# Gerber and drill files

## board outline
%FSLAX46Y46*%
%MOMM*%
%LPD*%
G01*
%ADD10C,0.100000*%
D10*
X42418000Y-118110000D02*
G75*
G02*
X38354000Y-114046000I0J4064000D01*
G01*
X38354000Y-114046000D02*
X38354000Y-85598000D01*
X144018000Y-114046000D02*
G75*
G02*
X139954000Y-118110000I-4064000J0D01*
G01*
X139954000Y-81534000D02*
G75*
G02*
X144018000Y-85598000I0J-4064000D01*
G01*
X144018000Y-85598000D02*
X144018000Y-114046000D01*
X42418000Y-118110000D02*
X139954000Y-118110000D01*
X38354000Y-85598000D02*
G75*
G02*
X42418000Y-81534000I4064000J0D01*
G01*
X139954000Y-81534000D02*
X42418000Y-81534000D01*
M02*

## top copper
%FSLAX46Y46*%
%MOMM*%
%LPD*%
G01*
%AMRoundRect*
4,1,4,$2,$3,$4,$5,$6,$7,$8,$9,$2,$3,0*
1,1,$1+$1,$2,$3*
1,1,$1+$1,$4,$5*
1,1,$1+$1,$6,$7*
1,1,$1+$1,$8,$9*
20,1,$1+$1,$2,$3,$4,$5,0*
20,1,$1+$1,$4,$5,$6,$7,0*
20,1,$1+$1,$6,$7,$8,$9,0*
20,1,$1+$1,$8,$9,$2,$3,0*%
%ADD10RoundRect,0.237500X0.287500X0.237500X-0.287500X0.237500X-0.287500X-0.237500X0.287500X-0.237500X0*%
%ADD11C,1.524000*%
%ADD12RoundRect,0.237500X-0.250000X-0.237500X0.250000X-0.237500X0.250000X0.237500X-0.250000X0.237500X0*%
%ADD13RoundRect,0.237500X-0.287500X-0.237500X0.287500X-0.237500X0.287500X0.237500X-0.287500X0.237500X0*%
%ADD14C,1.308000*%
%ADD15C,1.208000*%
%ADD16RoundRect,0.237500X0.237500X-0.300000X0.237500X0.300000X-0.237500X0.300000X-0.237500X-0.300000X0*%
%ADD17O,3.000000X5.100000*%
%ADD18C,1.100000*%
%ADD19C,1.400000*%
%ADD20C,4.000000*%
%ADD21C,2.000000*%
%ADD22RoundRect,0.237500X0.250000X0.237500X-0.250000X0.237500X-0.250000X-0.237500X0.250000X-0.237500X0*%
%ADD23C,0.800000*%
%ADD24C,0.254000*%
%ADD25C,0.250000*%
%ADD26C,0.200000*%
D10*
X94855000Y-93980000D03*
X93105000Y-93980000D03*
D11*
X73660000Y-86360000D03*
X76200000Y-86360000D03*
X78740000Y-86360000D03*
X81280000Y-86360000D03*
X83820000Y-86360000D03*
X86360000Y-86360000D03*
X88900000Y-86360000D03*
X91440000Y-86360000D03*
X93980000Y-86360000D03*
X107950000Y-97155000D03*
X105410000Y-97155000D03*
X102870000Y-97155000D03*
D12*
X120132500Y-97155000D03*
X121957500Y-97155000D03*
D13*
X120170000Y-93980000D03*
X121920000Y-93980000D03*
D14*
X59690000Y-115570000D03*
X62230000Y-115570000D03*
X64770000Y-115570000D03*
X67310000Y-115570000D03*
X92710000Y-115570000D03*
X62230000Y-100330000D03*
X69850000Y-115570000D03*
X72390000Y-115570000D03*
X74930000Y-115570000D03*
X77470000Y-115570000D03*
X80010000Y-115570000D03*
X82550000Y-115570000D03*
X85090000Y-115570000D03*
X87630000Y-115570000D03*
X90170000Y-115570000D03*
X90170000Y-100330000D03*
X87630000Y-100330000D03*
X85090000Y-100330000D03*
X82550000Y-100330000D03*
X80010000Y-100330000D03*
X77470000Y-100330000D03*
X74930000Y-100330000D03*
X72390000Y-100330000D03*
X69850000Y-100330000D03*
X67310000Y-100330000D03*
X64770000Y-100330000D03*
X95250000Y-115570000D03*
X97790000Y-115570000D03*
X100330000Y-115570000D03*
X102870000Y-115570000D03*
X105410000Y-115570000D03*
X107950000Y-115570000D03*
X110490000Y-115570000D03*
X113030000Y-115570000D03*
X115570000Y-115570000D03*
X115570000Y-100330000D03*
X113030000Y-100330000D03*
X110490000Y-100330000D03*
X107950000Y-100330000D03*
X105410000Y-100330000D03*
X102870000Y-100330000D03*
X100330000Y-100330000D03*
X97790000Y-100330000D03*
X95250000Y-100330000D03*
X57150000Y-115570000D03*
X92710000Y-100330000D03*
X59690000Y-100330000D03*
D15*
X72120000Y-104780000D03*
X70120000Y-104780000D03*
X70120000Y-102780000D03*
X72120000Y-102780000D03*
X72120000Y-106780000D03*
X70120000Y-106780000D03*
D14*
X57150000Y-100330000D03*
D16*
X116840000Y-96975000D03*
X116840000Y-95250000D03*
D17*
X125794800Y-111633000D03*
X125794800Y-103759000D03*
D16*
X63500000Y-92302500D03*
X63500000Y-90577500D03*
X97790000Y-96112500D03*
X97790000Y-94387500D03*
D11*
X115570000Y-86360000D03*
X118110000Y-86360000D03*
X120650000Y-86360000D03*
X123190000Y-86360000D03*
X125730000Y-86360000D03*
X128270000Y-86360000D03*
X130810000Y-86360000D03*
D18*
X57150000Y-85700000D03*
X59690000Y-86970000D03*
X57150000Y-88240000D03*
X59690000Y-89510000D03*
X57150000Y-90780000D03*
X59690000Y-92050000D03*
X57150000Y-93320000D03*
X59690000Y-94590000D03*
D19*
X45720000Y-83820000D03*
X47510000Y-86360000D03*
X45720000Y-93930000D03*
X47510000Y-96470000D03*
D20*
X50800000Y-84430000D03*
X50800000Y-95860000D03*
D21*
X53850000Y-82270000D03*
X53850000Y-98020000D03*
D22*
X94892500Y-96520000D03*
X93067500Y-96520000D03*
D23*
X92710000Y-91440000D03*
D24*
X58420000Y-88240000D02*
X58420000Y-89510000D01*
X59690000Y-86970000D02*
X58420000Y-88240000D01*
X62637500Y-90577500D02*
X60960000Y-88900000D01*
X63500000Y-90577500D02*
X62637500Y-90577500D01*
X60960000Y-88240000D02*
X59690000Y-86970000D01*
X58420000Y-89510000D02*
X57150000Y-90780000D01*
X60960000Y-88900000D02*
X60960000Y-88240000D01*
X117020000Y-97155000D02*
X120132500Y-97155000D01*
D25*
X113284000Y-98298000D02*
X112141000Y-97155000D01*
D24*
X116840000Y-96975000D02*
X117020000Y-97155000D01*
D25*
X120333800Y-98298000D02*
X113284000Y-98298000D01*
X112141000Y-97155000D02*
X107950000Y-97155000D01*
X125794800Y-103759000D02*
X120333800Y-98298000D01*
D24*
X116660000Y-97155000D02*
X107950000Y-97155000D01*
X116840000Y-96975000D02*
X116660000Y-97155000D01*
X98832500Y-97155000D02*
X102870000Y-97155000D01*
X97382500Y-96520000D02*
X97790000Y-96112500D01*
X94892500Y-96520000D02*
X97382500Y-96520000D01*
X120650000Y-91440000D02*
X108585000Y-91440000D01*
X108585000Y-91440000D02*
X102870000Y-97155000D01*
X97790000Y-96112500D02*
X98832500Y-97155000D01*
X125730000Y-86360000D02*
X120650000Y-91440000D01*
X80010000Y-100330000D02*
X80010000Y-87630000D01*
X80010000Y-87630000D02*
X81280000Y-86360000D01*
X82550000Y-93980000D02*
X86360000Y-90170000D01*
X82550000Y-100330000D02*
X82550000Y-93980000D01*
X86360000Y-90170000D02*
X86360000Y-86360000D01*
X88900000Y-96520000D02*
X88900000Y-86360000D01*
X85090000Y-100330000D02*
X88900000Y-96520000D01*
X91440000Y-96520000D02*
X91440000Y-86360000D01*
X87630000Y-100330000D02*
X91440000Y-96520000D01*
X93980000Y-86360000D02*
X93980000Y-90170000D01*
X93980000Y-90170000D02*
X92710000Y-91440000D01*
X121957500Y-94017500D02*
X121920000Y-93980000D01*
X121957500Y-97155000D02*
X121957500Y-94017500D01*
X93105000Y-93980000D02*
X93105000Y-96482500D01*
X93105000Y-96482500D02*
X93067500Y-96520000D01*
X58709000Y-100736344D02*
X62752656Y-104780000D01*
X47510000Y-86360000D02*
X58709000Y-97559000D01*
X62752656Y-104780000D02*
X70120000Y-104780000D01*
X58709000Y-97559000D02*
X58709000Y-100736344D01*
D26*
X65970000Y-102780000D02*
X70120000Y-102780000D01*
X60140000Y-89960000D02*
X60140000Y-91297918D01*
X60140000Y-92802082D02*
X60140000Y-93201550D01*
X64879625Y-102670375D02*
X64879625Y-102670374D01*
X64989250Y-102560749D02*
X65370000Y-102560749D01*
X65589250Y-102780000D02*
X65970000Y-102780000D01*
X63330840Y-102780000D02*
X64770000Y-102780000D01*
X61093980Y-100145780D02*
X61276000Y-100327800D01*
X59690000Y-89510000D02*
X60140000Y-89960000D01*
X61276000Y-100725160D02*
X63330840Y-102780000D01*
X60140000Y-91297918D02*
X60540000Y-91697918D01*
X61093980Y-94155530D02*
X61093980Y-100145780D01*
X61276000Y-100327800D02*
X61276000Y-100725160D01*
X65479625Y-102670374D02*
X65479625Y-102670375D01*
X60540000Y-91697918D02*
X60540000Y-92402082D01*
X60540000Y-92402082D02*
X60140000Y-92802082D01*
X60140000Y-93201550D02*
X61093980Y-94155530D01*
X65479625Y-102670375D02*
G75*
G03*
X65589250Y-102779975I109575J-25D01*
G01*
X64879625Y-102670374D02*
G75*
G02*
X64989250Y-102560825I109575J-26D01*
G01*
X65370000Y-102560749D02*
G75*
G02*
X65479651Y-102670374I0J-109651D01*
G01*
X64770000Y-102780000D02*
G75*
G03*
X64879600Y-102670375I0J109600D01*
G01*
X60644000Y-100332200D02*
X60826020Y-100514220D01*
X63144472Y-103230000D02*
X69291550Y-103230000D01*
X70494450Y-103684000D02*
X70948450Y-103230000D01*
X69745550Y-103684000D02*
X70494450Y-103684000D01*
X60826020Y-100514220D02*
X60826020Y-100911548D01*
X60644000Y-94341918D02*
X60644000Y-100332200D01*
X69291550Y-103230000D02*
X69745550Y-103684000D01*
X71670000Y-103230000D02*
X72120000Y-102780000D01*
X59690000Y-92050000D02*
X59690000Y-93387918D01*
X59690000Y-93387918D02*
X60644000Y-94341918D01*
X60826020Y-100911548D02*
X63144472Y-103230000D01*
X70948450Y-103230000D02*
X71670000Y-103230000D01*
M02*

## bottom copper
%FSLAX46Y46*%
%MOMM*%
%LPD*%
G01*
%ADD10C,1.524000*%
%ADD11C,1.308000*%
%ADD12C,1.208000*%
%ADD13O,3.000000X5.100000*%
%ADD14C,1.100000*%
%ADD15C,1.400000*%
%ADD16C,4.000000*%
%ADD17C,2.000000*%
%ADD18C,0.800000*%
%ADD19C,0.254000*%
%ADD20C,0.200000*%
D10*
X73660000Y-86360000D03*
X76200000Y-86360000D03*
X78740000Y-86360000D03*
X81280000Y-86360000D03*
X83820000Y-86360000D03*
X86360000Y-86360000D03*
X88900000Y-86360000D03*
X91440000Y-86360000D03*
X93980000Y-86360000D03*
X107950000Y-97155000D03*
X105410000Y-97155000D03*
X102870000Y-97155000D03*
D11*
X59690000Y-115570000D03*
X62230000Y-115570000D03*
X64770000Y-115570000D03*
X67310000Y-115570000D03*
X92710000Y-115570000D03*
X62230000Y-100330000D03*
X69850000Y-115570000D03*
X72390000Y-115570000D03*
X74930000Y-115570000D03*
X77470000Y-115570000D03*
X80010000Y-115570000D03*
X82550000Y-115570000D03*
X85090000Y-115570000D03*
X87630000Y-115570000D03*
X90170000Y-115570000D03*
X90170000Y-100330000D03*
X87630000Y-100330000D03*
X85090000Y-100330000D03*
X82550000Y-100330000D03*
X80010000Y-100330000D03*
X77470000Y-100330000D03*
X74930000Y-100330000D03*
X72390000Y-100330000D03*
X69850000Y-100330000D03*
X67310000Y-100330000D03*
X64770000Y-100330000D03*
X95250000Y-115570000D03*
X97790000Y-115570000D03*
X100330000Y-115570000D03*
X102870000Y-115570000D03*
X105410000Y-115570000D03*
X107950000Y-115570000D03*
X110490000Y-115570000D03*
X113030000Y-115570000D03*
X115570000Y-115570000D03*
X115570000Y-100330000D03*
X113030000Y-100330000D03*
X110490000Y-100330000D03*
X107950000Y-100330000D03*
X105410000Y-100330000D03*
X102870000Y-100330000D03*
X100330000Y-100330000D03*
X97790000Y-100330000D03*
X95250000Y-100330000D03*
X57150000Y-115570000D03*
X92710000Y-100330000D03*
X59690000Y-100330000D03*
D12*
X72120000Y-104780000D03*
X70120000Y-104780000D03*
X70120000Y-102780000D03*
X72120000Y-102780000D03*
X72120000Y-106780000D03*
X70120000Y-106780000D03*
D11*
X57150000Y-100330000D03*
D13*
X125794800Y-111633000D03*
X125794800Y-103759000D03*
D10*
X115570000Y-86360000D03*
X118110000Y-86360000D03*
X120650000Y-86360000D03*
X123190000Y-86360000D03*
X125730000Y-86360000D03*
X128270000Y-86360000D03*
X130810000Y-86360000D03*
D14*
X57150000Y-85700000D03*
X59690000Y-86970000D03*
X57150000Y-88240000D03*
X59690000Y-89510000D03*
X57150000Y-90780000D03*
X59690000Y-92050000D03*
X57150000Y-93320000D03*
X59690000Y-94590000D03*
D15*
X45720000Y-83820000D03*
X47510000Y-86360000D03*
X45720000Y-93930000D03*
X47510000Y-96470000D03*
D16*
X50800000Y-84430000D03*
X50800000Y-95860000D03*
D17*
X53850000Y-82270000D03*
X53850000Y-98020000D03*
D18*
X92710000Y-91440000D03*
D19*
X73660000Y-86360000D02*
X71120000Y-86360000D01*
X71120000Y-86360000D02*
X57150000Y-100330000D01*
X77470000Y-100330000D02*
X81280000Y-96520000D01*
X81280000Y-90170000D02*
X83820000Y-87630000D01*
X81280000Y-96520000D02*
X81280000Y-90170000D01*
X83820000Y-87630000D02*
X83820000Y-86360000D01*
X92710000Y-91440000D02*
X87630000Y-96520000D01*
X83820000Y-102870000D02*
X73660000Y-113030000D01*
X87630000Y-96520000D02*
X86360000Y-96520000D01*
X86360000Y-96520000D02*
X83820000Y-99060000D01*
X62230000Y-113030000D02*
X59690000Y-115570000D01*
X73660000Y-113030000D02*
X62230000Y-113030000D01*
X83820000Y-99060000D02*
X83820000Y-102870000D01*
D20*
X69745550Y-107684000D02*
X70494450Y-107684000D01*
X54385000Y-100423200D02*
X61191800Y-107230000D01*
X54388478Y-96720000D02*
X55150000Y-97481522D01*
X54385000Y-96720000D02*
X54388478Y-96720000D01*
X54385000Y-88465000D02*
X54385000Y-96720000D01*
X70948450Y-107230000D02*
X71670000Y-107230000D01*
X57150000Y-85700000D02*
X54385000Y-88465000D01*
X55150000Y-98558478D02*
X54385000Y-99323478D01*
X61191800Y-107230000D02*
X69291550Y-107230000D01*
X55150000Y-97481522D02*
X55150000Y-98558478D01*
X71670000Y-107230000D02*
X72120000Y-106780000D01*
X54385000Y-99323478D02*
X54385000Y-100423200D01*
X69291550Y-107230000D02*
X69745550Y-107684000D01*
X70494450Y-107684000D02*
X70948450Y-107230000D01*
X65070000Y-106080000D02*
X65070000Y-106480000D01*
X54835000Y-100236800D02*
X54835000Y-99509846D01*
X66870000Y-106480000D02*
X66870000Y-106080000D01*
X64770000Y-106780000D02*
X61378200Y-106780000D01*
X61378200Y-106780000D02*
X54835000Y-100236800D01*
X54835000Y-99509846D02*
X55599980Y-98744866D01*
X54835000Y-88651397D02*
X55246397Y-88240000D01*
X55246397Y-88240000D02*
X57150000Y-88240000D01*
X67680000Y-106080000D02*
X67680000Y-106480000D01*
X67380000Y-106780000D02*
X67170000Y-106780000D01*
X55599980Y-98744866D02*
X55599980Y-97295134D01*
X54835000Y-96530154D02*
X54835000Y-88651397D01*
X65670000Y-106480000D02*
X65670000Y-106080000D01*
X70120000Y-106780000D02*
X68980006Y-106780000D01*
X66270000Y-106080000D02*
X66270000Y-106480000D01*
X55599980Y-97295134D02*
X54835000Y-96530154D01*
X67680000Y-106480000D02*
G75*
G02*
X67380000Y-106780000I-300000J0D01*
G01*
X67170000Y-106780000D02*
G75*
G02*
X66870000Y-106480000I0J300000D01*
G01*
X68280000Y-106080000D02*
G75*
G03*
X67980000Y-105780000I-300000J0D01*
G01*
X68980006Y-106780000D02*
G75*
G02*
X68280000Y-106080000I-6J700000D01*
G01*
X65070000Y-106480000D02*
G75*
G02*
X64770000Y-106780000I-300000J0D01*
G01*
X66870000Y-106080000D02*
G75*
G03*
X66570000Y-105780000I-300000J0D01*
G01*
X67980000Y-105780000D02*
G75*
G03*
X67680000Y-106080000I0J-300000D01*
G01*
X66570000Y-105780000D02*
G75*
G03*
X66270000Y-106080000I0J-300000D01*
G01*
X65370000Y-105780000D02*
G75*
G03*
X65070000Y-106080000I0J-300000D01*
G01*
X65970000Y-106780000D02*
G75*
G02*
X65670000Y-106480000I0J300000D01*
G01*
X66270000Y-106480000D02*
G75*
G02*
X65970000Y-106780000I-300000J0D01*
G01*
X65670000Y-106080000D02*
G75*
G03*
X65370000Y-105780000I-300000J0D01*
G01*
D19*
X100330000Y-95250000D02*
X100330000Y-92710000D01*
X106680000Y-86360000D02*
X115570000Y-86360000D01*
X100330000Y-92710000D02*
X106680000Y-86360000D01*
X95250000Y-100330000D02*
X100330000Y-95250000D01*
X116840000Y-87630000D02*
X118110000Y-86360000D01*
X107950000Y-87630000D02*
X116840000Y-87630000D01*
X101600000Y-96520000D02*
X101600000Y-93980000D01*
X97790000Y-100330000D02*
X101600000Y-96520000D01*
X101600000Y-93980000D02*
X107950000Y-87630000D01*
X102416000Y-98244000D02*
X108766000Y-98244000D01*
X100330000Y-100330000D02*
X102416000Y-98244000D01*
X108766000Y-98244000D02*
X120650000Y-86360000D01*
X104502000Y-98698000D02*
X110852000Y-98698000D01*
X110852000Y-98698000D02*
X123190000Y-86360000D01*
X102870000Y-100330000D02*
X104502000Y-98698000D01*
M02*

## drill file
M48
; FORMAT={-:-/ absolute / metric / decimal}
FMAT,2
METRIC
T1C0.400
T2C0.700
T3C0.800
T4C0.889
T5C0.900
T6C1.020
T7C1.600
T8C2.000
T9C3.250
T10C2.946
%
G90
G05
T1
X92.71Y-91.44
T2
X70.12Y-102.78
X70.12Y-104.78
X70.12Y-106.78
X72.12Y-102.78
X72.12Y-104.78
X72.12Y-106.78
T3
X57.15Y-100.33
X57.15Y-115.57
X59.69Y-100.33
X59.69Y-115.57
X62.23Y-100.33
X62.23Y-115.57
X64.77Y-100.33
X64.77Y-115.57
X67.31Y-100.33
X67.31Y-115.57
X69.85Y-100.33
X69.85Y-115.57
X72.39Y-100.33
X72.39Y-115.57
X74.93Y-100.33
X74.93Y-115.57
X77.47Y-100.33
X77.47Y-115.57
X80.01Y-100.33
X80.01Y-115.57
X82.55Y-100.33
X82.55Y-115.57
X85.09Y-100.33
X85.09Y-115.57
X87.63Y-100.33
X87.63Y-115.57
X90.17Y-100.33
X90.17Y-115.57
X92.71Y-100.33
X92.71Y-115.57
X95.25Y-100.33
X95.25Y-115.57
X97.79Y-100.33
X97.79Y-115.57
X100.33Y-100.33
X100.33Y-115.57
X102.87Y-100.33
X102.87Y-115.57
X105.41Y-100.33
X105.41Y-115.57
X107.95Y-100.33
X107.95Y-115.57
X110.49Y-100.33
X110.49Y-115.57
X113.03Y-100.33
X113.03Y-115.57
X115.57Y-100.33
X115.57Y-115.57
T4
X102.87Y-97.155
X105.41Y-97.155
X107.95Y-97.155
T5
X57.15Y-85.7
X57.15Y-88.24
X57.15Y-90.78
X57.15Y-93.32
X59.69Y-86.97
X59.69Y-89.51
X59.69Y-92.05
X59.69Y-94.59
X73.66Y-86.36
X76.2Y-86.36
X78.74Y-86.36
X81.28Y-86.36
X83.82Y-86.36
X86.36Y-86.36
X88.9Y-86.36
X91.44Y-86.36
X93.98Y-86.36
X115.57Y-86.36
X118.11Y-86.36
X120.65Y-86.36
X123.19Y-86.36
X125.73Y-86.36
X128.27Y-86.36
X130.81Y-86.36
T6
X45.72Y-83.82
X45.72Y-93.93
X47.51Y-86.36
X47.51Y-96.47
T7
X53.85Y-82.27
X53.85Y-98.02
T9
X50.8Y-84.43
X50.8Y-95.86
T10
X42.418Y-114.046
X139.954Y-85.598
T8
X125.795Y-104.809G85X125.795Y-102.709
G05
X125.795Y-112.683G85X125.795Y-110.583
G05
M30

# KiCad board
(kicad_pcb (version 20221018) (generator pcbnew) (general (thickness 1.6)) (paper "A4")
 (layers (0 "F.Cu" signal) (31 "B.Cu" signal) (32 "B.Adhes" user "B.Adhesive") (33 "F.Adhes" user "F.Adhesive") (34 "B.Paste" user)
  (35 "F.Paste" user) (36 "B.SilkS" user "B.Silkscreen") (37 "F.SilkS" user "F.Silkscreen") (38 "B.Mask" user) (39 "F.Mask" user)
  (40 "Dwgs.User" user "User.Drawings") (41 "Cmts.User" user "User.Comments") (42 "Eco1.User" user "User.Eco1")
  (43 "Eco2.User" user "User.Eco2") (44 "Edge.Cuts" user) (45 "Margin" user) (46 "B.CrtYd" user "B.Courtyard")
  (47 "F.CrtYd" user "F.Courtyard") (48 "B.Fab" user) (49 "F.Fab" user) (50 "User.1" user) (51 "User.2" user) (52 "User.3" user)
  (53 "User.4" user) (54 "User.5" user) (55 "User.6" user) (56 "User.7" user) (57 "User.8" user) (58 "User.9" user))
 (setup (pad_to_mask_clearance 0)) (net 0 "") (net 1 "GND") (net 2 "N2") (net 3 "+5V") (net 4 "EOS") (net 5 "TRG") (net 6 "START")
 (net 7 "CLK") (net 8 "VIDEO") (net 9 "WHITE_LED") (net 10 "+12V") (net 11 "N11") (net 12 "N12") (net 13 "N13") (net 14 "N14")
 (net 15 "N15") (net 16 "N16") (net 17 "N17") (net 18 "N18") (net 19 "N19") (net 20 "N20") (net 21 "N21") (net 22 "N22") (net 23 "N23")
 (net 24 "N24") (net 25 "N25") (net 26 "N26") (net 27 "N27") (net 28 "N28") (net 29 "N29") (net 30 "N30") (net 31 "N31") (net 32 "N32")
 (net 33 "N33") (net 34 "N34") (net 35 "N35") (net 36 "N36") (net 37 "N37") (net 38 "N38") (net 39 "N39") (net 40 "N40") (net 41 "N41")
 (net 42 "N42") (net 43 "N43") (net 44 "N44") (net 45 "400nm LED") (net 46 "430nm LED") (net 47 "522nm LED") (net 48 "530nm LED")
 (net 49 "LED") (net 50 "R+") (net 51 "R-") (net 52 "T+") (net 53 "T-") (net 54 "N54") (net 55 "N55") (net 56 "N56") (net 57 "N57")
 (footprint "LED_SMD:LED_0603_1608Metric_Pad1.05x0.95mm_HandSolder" (layer "F.Cu") (at 93.98 93.98 180)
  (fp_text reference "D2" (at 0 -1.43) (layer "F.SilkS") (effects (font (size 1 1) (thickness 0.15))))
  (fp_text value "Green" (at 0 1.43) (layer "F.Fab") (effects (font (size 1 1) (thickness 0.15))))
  (pad "1" smd roundrect (at -0.875 0 180) (size 1.05 0.95) (layers "F.Cu" "F.Paste" "F.Mask") (roundrect_rratio 0.25) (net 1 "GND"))
  (pad "2" smd roundrect (at 0.875 0 180) (size 1.05 0.95) (layers "F.Cu" "F.Paste" "F.Mask") (roundrect_rratio 0.25) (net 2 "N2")))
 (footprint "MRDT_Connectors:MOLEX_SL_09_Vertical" (layer "F.Cu") (at 73.66 86.36)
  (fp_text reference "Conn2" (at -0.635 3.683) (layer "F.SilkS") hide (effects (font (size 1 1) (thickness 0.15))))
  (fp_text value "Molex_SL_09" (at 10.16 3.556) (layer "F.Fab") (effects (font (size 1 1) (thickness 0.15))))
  (pad "1" thru_hole circle (at 0 0) (size 1.524 1.524) (drill 0.9) (layers "*.Cu" "*.Mask") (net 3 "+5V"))
  (pad "2" thru_hole circle (at 2.54 0) (size 1.524 1.524) (drill 0.9) (layers "*.Cu" "*.Mask") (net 1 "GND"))
  (pad "3" thru_hole circle (at 5.08 0) (size 1.524 1.524) (drill 0.9) (layers "*.Cu" "*.Mask") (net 1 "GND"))
  (pad "4" thru_hole circle (at 7.62 0) (size 1.524 1.524) (drill 0.9) (layers "*.Cu" "*.Mask") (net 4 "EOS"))
  (pad "5" thru_hole circle (at 10.16 0) (size 1.524 1.524) (drill 0.9) (layers "*.Cu" "*.Mask") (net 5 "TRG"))
  (pad "6" thru_hole circle (at 12.7 0) (size 1.524 1.524) (drill 0.9) (layers "*.Cu" "*.Mask") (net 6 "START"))
  (pad "7" thru_hole circle (at 15.24 0) (size 1.524 1.524) (drill 0.9) (layers "*.Cu" "*.Mask") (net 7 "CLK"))
  (pad "8" thru_hole circle (at 17.78 0) (size 1.524 1.524) (drill 0.9) (layers "*.Cu" "*.Mask") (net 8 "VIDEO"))
  (pad "9" thru_hole circle (at 20.32 0) (size 1.524 1.524) (drill 0.9) (layers "*.Cu" "*.Mask") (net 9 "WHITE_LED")))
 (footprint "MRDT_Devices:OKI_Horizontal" (layer "F.Cu") (at 107.95 97.155 180)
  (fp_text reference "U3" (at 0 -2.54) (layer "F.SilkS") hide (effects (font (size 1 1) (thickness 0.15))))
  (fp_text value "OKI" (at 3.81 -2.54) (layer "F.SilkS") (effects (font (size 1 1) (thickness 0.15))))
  (pad "1" thru_hole circle (at 0 0 180) (size 1.524 1.524) (drill 0.889) (layers "*.Cu" "*.Mask") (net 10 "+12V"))
  (pad "2" thru_hole circle (at 2.54 0 180) (size 1.524 1.524) (drill 0.889) (layers "*.Cu" "*.Mask") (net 1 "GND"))
  (pad "3" thru_hole circle (at 5.08 0 180) (size 1.524 1.524) (drill 0.889) (layers "*.Cu" "*.Mask") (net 3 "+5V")))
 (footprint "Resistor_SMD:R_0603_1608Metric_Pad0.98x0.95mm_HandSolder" (layer "F.Cu") (at 121.045 97.155)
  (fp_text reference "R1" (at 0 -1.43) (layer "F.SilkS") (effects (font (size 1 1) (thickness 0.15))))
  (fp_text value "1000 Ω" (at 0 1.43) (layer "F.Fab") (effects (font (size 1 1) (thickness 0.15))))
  (pad "1" smd roundrect (at -0.9125 0) (size 0.975 0.95) (layers "F.Cu" "F.Paste" "F.Mask") (roundrect_rratio 0.25) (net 10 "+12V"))
  (pad "2" smd roundrect (at 0.9125 0) (size 0.975 0.95) (layers "F.Cu" "F.Paste" "F.Mask") (roundrect_rratio 0.25) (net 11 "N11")))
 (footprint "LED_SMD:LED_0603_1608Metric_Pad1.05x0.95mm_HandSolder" (layer "F.Cu") (at 121.045 93.98)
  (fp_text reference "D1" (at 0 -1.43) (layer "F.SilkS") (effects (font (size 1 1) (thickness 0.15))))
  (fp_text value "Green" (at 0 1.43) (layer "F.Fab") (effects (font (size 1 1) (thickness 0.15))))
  (pad "1" smd roundrect (at -0.875 0) (size 1.05 0.95) (layers "F.Cu" "F.Paste" "F.Mask") (roundrect_rratio 0.25) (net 1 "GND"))
  (pad "2" smd roundrect (at 0.875 0) (size 1.05 0.95) (layers "F.Cu" "F.Paste" "F.Mask") (roundrect_rratio 0.25) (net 11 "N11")))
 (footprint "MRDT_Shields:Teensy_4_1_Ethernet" (layer "F.Cu") (at 86.36 107.95)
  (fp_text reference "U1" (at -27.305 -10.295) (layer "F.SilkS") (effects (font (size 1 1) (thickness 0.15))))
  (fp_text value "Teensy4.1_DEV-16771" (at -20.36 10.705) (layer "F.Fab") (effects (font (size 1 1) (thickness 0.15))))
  (pad "0" thru_hole circle (at -26.67 7.62) (size 1.308 1.308) (drill 0.8) (layers "*.Cu" "*.Mask") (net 9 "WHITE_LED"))
  (pad "1" thru_hole circle (at -24.13 7.62) (size 1.308 1.308) (drill 0.8) (layers "*.Cu" "*.Mask") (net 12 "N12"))
  (pad "2" thru_hole circle (at -21.59 7.62) (size 1.308 1.308) (drill 0.8) (layers "*.Cu" "*.Mask") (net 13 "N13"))
  (pad "3" thru_hole circle (at -19.05 7.62) (size 1.308 1.308) (drill 0.8) (layers "*.Cu" "*.Mask") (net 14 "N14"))
  (pad "3.3V_1" thru_hole circle (at 6.35 7.62) (size 1.308 1.308) (drill 0.8) (layers "*.Cu" "*.Mask") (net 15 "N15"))
  (pad "3.3V_2" thru_hole circle (at -24.13 -7.62) (size 1.308 1.308) (drill 0.8) (layers "*.Cu" "*.Mask") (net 15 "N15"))
  (pad "4" thru_hole circle (at -16.51 7.62) (size 1.308 1.308) (drill 0.8) (layers "*.Cu" "*.Mask") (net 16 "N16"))
  (pad "5" thru_hole circle (at -13.97 7.62) (size 1.308 1.308) (drill 0.8) (layers "*.Cu" "*.Mask") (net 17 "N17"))
  (pad "6" thru_hole circle (at -11.43 7.62) (size 1.308 1.308) (drill 0.8) (layers "*.Cu" "*.Mask") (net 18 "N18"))
  (pad "7" thru_hole circle (at -8.89 7.62) (size 1.308 1.308) (drill 0.8) (layers "*.Cu" "*.Mask") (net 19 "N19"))
  (pad "8" thru_hole circle (at -6.35 7.62) (size 1.308 1.308) (drill 0.8) (layers "*.Cu" "*.Mask") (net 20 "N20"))
  (pad "9" thru_hole circle (at -3.81 7.62) (size 1.308 1.308) (drill 0.8) (layers "*.Cu" "*.Mask") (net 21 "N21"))
  (pad "10" thru_hole circle (at -1.27 7.62) (size 1.308 1.308) (drill 0.8) (layers "*.Cu" "*.Mask") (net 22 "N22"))
  (pad "11" thru_hole circle (at 1.27 7.62) (size 1.308 1.308) (drill 0.8) (layers "*.Cu" "*.Mask") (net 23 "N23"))
  (pad "12" thru_hole circle (at 3.81 7.62) (size 1.308 1.308) (drill 0.8) (layers "*.Cu" "*.Mask") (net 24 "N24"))
  (pad "13" thru_hole circle (at 3.81 -7.62) (size 1.308 1.308) (drill 0.8) (layers "*.Cu" "*.Mask") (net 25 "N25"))
  (pad "14" thru_hole circle (at 1.27 -7.62) (size 1.308 1.308) (drill 0.8) (layers "*.Cu" "*.Mask") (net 8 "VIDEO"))
  (pad "15" thru_hole circle (at -1.27 -7.62) (size 1.308 1.308) (drill 0.8) (layers "*.Cu" "*.Mask") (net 7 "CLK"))
  (pad "16" thru_hole circle (at -3.81 -7.62) (size 1.308 1.308) (drill 0.8) (layers "*.Cu" "*.Mask") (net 6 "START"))
  (pad "17" thru_hole circle (at -6.35 -7.62) (size 1.308 1.308) (drill 0.8) (layers "*.Cu" "*.Mask") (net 4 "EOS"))
  (pad "18" thru_hole circle (at -8.89 -7.62) (size 1.308 1.308) (drill 0.8) (layers "*.Cu" "*.Mask") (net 5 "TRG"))
  (pad "19" thru_hole circle (at -11.43 -7.62) (size 1.308 1.308) (drill 0.8) (layers "*.Cu" "*.Mask") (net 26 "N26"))
  (pad "20" thru_hole circle (at -13.97 -7.62) (size 1.308 1.308) (drill 0.8) (layers "*.Cu" "*.Mask") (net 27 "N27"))
  (pad "21" thru_hole circle (at -16.51 -7.62) (size 1.308 1.308) (drill 0.8) (layers "*.Cu" "*.Mask") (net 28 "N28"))
  (pad "22" thru_hole circle (at -19.05 -7.62) (size 1.308 1.308) (drill 0.8) (layers "*.Cu" "*.Mask") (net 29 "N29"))
  (pad "23" thru_hole circle (at -21.59 -7.62) (size 1.308 1.308) (drill 0.8) (layers "*.Cu" "*.Mask") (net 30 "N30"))
  (pad "24" thru_hole circle (at 8.89 7.62) (size 1.308 1.308) (drill 0.8) (layers "*.Cu" "*.Mask") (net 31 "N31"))
  (pad "25" thru_hole circle (at 11.43 7.62) (size 1.308 1.308) (drill 0.8) (layers "*.Cu" "*.Mask") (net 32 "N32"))
  (pad "26" thru_hole circle (at 13.97 7.62) (size 1.308 1.308) (drill 0.8) (layers "*.Cu" "*.Mask") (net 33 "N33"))
  (pad "27" thru_hole circle (at 16.51 7.62) (size 1.308 1.308) (drill 0.8) (layers "*.Cu" "*.Mask") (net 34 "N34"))
  (pad "28" thru_hole circle (at 19.05 7.62) (size 1.308 1.308) (drill 0.8) (layers "*.Cu" "*.Mask") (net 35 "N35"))
  (pad "29" thru_hole circle (at 21.59 7.62) (size 1.308 1.308) (drill 0.8) (layers "*.Cu" "*.Mask") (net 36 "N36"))
  (pad "30" thru_hole circle (at 24.13 7.62) (size 1.308 1.308) (drill 0.8) (layers "*.Cu" "*.Mask") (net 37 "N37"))
  (pad "31" thru_hole circle (at 26.67 7.62) (size 1.308 1.308) (drill 0.8) (layers "*.Cu" "*.Mask") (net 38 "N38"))
  (pad "32" thru_hole circle (at 29.21 7.62) (size 1.308 1.308) (drill 0.8) (layers "*.Cu" "*.Mask") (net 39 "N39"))
  (pad "33" thru_hole circle (at 29.21 -7.62) (size 1.308 1.308) (drill 0.8) (layers "*.Cu" "*.Mask") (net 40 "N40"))
  (pad "34" thru_hole circle (at 26.67 -7.62) (size 1.308 1.308) (drill 0.8) (layers "*.Cu" "*.Mask") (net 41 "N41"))
  (pad "35" thru_hole circle (at 24.13 -7.62) (size 1.308 1.308) (drill 0.8) (layers "*.Cu" "*.Mask") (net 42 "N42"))
  (pad "36" thru_hole circle (at 21.59 -7.62) (size 1.308 1.308) (drill 0.8) (layers "*.Cu" "*.Mask") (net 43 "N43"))
  (pad "37" thru_hole circle (at 19.05 -7.62) (size 1.308 1.308) (drill 0.8) (layers "*.Cu" "*.Mask") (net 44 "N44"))
  (pad "38" thru_hole circle (at 16.51 -7.62) (size 1.308 1.308) (drill 0.8) (layers "*.Cu" "*.Mask") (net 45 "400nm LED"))
  (pad "39" thru_hole circle (at 13.97 -7.62) (size 1.308 1.308) (drill 0.8) (layers "*.Cu" "*.Mask") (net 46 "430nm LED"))
  (pad "40" thru_hole circle (at 11.43 -7.62) (size 1.308 1.308) (drill 0.8) (layers "*.Cu" "*.Mask") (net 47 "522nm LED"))
  (pad "41" thru_hole circle (at 8.89 -7.62) (size 1.308 1.308) (drill 0.8) (layers "*.Cu" "*.Mask") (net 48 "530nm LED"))
  (pad "GND1" thru_hole circle (at -29.21 7.62) (size 1.308 1.308) (drill 0.8) (layers "*.Cu" "*.Mask") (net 1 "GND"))
  (pad "GND2" thru_hole circle (at 6.35 -7.62) (size 1.308 1.308) (drill 0.8) (layers "*.Cu" "*.Mask") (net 1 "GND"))
  (pad "GND3" thru_hole circle (at -26.67 -7.62) (size 1.308 1.308) (drill 0.8) (layers "*.Cu" "*.Mask") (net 1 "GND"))
  (pad "GND5" thru_hole circle (at -14.24 -3.17) (size 1.208 1.208) (drill 0.7) (layers "*.Cu" "*.Mask") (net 1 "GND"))
  (pad "LED" thru_hole circle (at -16.24 -3.17) (size 1.208 1.208) (drill 0.7) (layers "*.Cu" "*.Mask") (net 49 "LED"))
  (pad "R+" thru_hole circle (at -16.24 -5.17) (size 1.208 1.208) (drill 0.7) (layers "*.Cu" "*.Mask") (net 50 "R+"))
  (pad "R-" thru_hole circle (at -14.24 -5.17) (size 1.208 1.208) (drill 0.7) (layers "*.Cu" "*.Mask") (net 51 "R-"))
  (pad "T+" thru_hole circle (at -14.24 -1.17) (size 1.208 1.208) (drill 0.7) (layers "*.Cu" "*.Mask") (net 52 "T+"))
  (pad "T-" thru_hole circle (at -16.24 -1.17) (size 1.208 1.208) (drill 0.7) (layers "*.Cu" "*.Mask") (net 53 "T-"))
  (pad "VIN" thru_hole circle (at -29.21 -7.62) (size 1.308 1.308) (drill 0.8) (layers "*.Cu" "*.Mask") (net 3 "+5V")))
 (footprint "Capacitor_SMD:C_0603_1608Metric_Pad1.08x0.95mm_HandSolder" (layer "F.Cu") (at 116.84 96.1125 90)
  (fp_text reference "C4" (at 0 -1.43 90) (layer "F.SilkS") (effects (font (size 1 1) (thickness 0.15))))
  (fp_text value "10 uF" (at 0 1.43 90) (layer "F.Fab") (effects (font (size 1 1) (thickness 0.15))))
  (pad "1" smd roundrect (at -0.8625 0 90) (size 1.075 0.95) (layers "F.Cu" "F.Paste" "F.Mask") (roundrect_rratio 0.25) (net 10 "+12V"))
  (pad "2" smd roundrect (at 0.8625 0 90) (size 1.075 0.95) (layers "F.Cu" "F.Paste" "F.Mask") (roundrect_rratio 0.25) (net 1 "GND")))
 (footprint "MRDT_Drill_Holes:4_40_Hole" (layer "F.Cu") (at 139.954 85.598) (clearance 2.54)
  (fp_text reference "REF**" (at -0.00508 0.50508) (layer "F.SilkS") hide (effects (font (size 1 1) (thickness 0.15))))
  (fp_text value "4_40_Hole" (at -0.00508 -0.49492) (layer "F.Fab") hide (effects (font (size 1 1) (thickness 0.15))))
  (pad "" np_thru_hole circle (at 0 0) (size 2.9464 2.9464) (drill 2.9464) (layers "*.Cu" "*.Mask") (clearance 2.5)))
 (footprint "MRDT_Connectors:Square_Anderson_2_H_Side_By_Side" (layer "F.Cu") (at 125.4202 112.183 180)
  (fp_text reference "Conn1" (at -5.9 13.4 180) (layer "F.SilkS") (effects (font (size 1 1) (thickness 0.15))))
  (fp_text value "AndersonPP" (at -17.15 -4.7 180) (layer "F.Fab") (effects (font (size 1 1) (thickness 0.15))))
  (pad "1" thru_hole oval (at -0.3746 0.55 180) (size 3 5.1) (drill oval 2 4.1) (layers "*.Cu" "*.Mask" "F.Paste") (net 1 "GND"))
  (pad "2" thru_hole oval (at -0.3746 8.424 180) (size 3 5.1) (drill oval 2 4.1) (layers "*.Cu" "*.Mask" "F.Paste") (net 10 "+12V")))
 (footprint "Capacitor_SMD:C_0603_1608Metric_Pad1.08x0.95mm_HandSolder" (layer "F.Cu") (at 63.5 91.44 90)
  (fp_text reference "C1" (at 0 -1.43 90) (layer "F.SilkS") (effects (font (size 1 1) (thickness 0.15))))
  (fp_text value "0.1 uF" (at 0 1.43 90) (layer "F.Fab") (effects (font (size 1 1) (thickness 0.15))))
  (pad "1" smd roundrect (at -0.8625 0 90) (size 1.075 0.95) (layers "F.Cu" "F.Paste" "F.Mask") (roundrect_rratio 0.25) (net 1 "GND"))
  (pad "2" smd roundrect (at 0.8625 0 90) (size 1.075 0.95) (layers "F.Cu" "F.Paste" "F.Mask") (roundrect_rratio 0.25) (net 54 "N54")))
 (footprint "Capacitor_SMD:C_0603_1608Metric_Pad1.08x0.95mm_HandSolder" (layer "F.Cu") (at 97.79 95.25 90)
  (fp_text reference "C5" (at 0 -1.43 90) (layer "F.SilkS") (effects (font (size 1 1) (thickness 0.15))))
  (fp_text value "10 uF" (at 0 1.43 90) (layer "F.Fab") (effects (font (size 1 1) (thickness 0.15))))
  (pad "1" smd roundrect (at -0.8625 0 90) (size 1.075 0.95) (layers "F.Cu" "F.Paste" "F.Mask") (roundrect_rratio 0.25) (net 3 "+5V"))
  (pad "2" smd roundrect (at 0.8625 0 90) (size 1.075 0.95) (layers "F.Cu" "F.Paste" "F.Mask") (roundrect_rratio 0.25) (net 1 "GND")))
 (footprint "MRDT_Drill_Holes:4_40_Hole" (layer "F.Cu") (at 42.418 114.046) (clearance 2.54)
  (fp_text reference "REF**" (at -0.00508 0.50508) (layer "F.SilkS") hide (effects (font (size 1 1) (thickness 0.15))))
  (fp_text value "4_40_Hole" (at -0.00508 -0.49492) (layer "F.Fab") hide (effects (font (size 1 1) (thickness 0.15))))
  (pad "" np_thru_hole circle (at 0 0) (size 2.9464 2.9464) (drill 2.9464) (layers "*.Cu" "*.Mask") (clearance 2.5)))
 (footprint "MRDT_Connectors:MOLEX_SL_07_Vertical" (layer "F.Cu") (at 115.57 86.36)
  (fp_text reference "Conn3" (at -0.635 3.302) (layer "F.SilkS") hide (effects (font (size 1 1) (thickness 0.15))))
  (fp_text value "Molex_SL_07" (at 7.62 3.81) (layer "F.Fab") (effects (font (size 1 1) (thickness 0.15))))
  (pad "1" thru_hole circle (at 0 0) (size 1.524 1.524) (drill 0.9) (layers "*.Cu" "*.Mask") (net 48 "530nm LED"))
  (pad "2" thru_hole circle (at 2.54 0) (size 1.524 1.524) (drill 0.9) (layers "*.Cu" "*.Mask") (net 47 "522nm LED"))
  (pad "3" thru_hole circle (at 5.08 0) (size 1.524 1.524) (drill 0.9) (layers "*.Cu" "*.Mask") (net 46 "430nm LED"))
  (pad "4" thru_hole circle (at 7.62 0) (size 1.524 1.524) (drill 0.9) (layers "*.Cu" "*.Mask") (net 45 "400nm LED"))
  (pad "5" thru_hole circle (at 10.16 0) (size 1.524 1.524) (drill 0.9) (layers "*.Cu" "*.Mask") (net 3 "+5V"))
  (pad "6" thru_hole circle (at 12.7 0) (size 1.524 1.524) (drill 0.9) (layers "*.Cu" "*.Mask") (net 1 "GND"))
  (pad "7" thru_hole circle (at 15.24 0) (size 1.524 1.524) (drill 0.9) (layers "*.Cu" "*.Mask") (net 1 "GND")))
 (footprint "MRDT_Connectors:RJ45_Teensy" (layer "F.Cu") (at 37.8 90.27 -90)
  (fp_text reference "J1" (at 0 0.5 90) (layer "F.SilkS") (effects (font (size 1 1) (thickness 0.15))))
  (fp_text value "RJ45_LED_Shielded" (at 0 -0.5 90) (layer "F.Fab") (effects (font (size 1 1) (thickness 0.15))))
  (pad "1" thru_hole circle (at -4.57 -19.35 270) (size 1.1 1.1) (drill 0.9) (layers "*.Cu" "*.Mask") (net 52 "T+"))
  (pad "2" thru_hole circle (at -3.3 -21.89 270) (size 1.1 1.1) (drill 0.9) (layers "*.Cu" "*.Mask") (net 54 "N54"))
  (pad "3" thru_hole circle (at -2.03 -19.35 270) (size 1.1 1.1) (drill 0.9) (layers "*.Cu" "*.Mask") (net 53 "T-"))
  (pad "4" thru_hole circle (at -0.76 -21.89 270) (size 1.1 1.1) (drill 0.9) (layers "*.Cu" "*.Mask") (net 50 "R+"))
  (pad "5" thru_hole circle (at 0.51 -19.35 270) (size 1.1 1.1) (drill 0.9) (layers "*.Cu" "*.Mask") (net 54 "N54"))
  (pad "6" thru_hole circle (at 1.78 -21.89 270) (size 1.1 1.1) (drill 0.9) (layers "*.Cu" "*.Mask") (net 51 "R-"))
  (pad "7" thru_hole circle (at 3.05 -19.35 270) (size 1.1 1.1) (drill 0.9) (layers "*.Cu" "*.Mask") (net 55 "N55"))
  (pad "8" thru_hole circle (at 4.32 -21.89 270) (size 1.1 1.1) (drill 0.9) (layers "*.Cu" "*.Mask") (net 1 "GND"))
  (pad "9" thru_hole circle (at -6.45 -7.92 270) (size 1.4 1.4) (drill 1.02) (layers "*.Cu" "*.Mask") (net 1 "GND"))
  (pad "10" thru_hole circle (at -3.91 -9.71 270) (size 1.4 1.4) (drill 1.02) (layers "*.Cu" "*.Mask") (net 49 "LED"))
  (pad "11" thru_hole circle (at 3.66 -7.92 270) (size 1.4 1.4) (drill 1.02) (layers "*.Cu" "*.Mask") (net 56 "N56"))
  (pad "12" thru_hole circle (at 6.2 -9.71 270) (size 1.4 1.4) (drill 1.02) (layers "*.Cu" "*.Mask") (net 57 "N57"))
  (pad "13" thru_hole circle (at -5.84 -13 270) (size 4 4) (drill 3.25) (layers "*.Cu" "*.Mask"))
  (pad "14" thru_hole circle (at 5.59 -13 270) (size 4 4) (drill 3.25) (layers "*.Cu" "*.Mask"))
  (pad "SH" thru_hole circle (at -8 -16.05 270) (size 2 2) (drill 1.6) (layers "*.Cu" "*.Mask") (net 1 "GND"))
  (pad "SH" thru_hole circle (at 7.75 -16.05 270) (size 2 2) (drill 1.6) (layers "*.Cu" "*.Mask") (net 1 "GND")))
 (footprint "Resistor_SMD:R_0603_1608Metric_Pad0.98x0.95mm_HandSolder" (layer "F.Cu") (at 93.98 96.52 180)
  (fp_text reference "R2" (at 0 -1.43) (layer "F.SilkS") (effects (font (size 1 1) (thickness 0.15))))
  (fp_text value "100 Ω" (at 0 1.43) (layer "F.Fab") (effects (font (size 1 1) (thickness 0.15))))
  (pad "1" smd roundrect (at -0.9125 0 180) (size 0.975 0.95) (layers "F.Cu" "F.Paste" "F.Mask") (roundrect_rratio 0.25) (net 3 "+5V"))
  (pad "2" smd roundrect (at 0.9125 0 180) (size 0.975 0.95) (layers "F.Cu" "F.Paste" "F.Mask") (roundrect_rratio 0.25) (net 2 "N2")))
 (gr_arc (start 42.418 118.11) (mid 39.544318 116.919682) (end 38.354 114.046) (stroke (width 0.1) (type default)) (layer "Edge.Cuts"))
 (gr_line (start 38.354 114.046) (end 38.354 85.598) (stroke (width 0.1) (type default)) (layer "Edge.Cuts"))
 (gr_arc (start 144.018 114.046) (mid 142.827683 116.919683) (end 139.954 118.11) (stroke (width 0.1) (type default)) (layer "Edge.Cuts"))
 (gr_arc (start 139.954 81.534) (mid 142.827682 82.724318) (end 144.018 85.598) (stroke (width 0.1) (type default)) (layer "Edge.Cuts"))
 (gr_line (start 144.018 85.598) (end 144.018 114.046) (stroke (width 0.1) (type default)) (layer "Edge.Cuts"))
 (gr_line (start 42.418 118.11) (end 139.954 118.11) (stroke (width 0.1) (type default)) (layer "Edge.Cuts"))
 (gr_arc (start 38.354 85.598) (mid 39.544317 82.724317) (end 42.418 81.534) (stroke (width 0.1) (type default)) (layer "Edge.Cuts"))
 (gr_line (start 139.954 81.534) (end 42.418 81.534) (stroke (width 0.1) (type default)) (layer "Edge.Cuts"))
 (segment (start 58.42 88.24) (end 58.42 89.51) (width 0.254) (layer "F.Cu") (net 54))
 (segment (start 59.69 86.97) (end 58.42 88.24) (width 0.254) (layer "F.Cu") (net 54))
 (segment (start 62.6375 90.5775) (end 60.96 88.9) (width 0.254) (layer "F.Cu") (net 54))
 (segment (start 63.5 90.5775) (end 62.6375 90.5775) (width 0.254) (layer "F.Cu") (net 54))
 (segment (start 60.96 88.24) (end 59.69 86.97) (width 0.254) (layer "F.Cu") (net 54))
 (segment (start 58.42 89.51) (end 57.15 90.78) (width 0.254) (layer "F.Cu") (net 54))
 (segment (start 60.96 88.9) (end 60.96 88.24) (width 0.254) (layer "F.Cu") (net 54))
 (segment (start 117.02 97.155) (end 120.1325 97.155) (width 0.254) (layer "F.Cu") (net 10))
 (segment (start 113.284 98.298) (end 112.141 97.155) (width 0.25) (layer "F.Cu") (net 10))
 (segment (start 116.84 96.975) (end 117.02 97.155) (width 0.254) (layer "F.Cu") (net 10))
 (segment (start 120.3338 98.298) (end 113.284 98.298) (width 0.25) (layer "F.Cu") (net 10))
 (segment (start 112.141 97.155) (end 107.95 97.155) (width 0.25) (layer "F.Cu") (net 10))
 (segment (start 125.7948 103.759) (end 120.3338 98.298) (width 0.25) (layer "F.Cu") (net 10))
 (segment (start 116.66 97.155) (end 107.95 97.155) (width 0.254) (layer "F.Cu") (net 10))
 (segment (start 116.84 96.975) (end 116.66 97.155) (width 0.254) (layer "F.Cu") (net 10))
 (segment (start 98.8325 97.155) (end 102.87 97.155) (width 0.254) (layer "F.Cu") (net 3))
 (segment (start 97.3825 96.52) (end 97.79 96.1125) (width 0.254) (layer "F.Cu") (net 3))
 (segment (start 94.8925 96.52) (end 97.3825 96.52) (width 0.254) (layer "F.Cu") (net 3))
 (segment (start 120.65 91.44) (end 108.585 91.44) (width 0.254) (layer "F.Cu") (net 3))
 (segment (start 108.585 91.44) (end 102.87 97.155) (width 0.254) (layer "F.Cu") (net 3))
 (segment (start 97.79 96.1125) (end 98.8325 97.155) (width 0.254) (layer "F.Cu") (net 3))
 (segment (start 125.73 86.36) (end 120.65 91.44) (width 0.254) (layer "F.Cu") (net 3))
 (segment (start 73.66 86.36) (end 71.12 86.36) (width 0.254) (layer "B.Cu") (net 3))
 (segment (start 71.12 86.36) (end 57.15 100.33) (width 0.254) (layer "B.Cu") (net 3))
 (segment (start 80.01 100.33) (end 80.01 87.63) (width 0.254) (layer "F.Cu") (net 4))
 (segment (start 80.01 87.63) (end 81.28 86.36) (width 0.254) (layer "F.Cu") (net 4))
 (segment (start 77.47 100.33) (end 81.28 96.52) (width 0.254) (layer "B.Cu") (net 5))
 (segment (start 81.28 90.17) (end 83.82 87.63) (width 0.254) (layer "B.Cu") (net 5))
 (segment (start 81.28 96.52) (end 81.28 90.17) (width 0.254) (layer "B.Cu") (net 5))
 (segment (start 83.82 87.63) (end 83.82 86.36) (width 0.254) (layer "B.Cu") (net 5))
 (segment (start 82.55 93.98) (end 86.36 90.17) (width 0.254) (layer "F.Cu") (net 6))
 (segment (start 82.55 100.33) (end 82.55 93.98) (width 0.254) (layer "F.Cu") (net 6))
 (segment (start 86.36 90.17) (end 86.36 86.36) (width 0.254) (layer "F.Cu") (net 6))
 (segment (start 88.9 96.52) (end 88.9 86.36) (width 0.254) (layer "F.Cu") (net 7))
 (segment (start 85.09 100.33) (end 88.9 96.52) (width 0.254) (layer "F.Cu") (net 7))
 (segment (start 91.44 96.52) (end 91.44 86.36) (width 0.254) (layer "F.Cu") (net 8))
 (segment (start 87.63 100.33) (end 91.44 96.52) (width 0.254) (layer "F.Cu") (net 8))
 (segment (start 93.98 86.36) (end 93.98 90.17) (width 0.254) (layer "F.Cu") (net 9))
 (segment (start 93.98 90.17) (end 92.71 91.44) (width 0.254) (layer "F.Cu") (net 9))
 (via (at 92.71 91.44) (size 0.8) (drill 0.4) (layers "F.Cu" "B.Cu") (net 9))
 (segment (start 92.71 91.44) (end 87.63 96.52) (width 0.254) (layer "B.Cu") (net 9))
 (segment (start 83.82 102.87) (end 73.66 113.03) (width 0.254) (layer "B.Cu") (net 9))
 (segment (start 87.63 96.52) (end 86.36 96.52) (width 0.254) (layer "B.Cu") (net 9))
 (segment (start 86.36 96.52) (end 83.82 99.06) (width 0.254) (layer "B.Cu") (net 9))
 (segment (start 62.23 113.03) (end 59.69 115.57) (width 0.254) (layer "B.Cu") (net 9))
 (segment (start 73.66 113.03) (end 62.23 113.03) (width 0.254) (layer "B.Cu") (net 9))
 (segment (start 83.82 99.06) (end 83.82 102.87) (width 0.254) (layer "B.Cu") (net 9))
 (segment (start 121.9575 94.0175) (end 121.92 93.98) (width 0.254) (layer "F.Cu") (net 11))
 (segment (start 121.9575 97.155) (end 121.9575 94.0175) (width 0.254) (layer "F.Cu") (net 11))
 (segment (start 93.105 93.98) (end 93.105 96.4825) (width 0.254) (layer "F.Cu") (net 2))
 (segment (start 93.105 96.4825) (end 93.0675 96.52) (width 0.254) (layer "F.Cu") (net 2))
 (segment (start 58.709 100.736344) (end 62.752656 104.78) (width 0.254) (layer "F.Cu") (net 49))
 (segment (start 47.51 86.36) (end 58.709 97.559) (width 0.254) (layer "F.Cu") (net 49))
 (segment (start 62.752656 104.78) (end 70.12 104.78) (width 0.254) (layer "F.Cu") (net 49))
 (segment (start 58.709 97.559) (end 58.709 100.736344) (width 0.254) (layer "F.Cu") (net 49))
 (segment (start 69.74555 107.684) (end 70.49445 107.684) (width 0.2) (layer "B.Cu") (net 52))
 (segment (start 54.385 100.4232) (end 61.1918 107.23) (width 0.2) (layer "B.Cu") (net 52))
 (segment (start 54.388478 96.72) (end 55.15 97.481522) (width 0.2) (layer "B.Cu") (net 52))
 (segment (start 54.385 96.72) (end 54.388478 96.72) (width 0.2) (layer "B.Cu") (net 52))
 (segment (start 54.385 88.465) (end 54.385 96.72) (width 0.2) (layer "B.Cu") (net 52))
 (segment (start 70.94845 107.23) (end 71.67 107.23) (width 0.2) (layer "B.Cu") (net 52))
 (segment (start 57.15 85.7) (end 54.385 88.465) (width 0.2) (layer "B.Cu") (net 52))
 (segment (start 55.15 98.558478) (end 54.385 99.323478) (width 0.2) (layer "B.Cu") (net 52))
 (segment (start 61.1918 107.23) (end 69.29155 107.23) (width 0.2) (layer "B.Cu") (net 52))
 (segment (start 55.15 97.481522) (end 55.15 98.558478) (width 0.2) (layer "B.Cu") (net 52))
 (segment (start 71.67 107.23) (end 72.12 106.78) (width 0.2) (layer "B.Cu") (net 52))
 (segment (start 54.385 99.323478) (end 54.385 100.4232) (width 0.2) (layer "B.Cu") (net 52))
 (segment (start 69.29155 107.23) (end 69.74555 107.684) (width 0.2) (layer "B.Cu") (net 52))
 (segment (start 70.49445 107.684) (end 70.94845 107.23) (width 0.2) (layer "B.Cu") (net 52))
 (segment (start 65.07 106.08) (end 65.07 106.48) (width 0.2) (layer "B.Cu") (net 53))
 (segment (start 54.835 100.2368) (end 54.835 99.509846) (width 0.2) (layer "B.Cu") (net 53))
 (segment (start 66.87 106.48) (end 66.87 106.08) (width 0.2) (layer "B.Cu") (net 53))
 (segment (start 64.77 106.78) (end 61.3782 106.78) (width 0.2) (layer "B.Cu") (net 53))
 (segment (start 61.3782 106.78) (end 54.835 100.2368) (width 0.2) (layer "B.Cu") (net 53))
 (segment (start 54.835 99.509846) (end 55.59998 98.744866) (width 0.2) (layer "B.Cu") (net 53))
 (segment (start 54.835 88.651397) (end 55.246397 88.24) (width 0.2) (layer "B.Cu") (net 53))
 (segment (start 55.246397 88.24) (end 57.15 88.24) (width 0.2) (layer "B.Cu") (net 53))
 (segment (start 67.68 106.08) (end 67.68 106.48) (width 0.2) (layer "B.Cu") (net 53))
 (segment (start 67.38 106.78) (end 67.17 106.78) (width 0.2) (layer "B.Cu") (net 53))
 (segment (start 55.59998 98.744866) (end 55.59998 97.295134) (width 0.2) (layer "B.Cu") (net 53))
 (segment (start 54.835 96.530154) (end 54.835 88.651397) (width 0.2) (layer "B.Cu") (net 53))
 (segment (start 65.67 106.48) (end 65.67 106.08) (width 0.2) (layer "B.Cu") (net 53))
 (segment (start 70.12 106.78) (end 68.980006 106.78) (width 0.2) (layer "B.Cu") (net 53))
 (segment (start 66.27 106.08) (end 66.27 106.48) (width 0.2) (layer "B.Cu") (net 53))
 (segment (start 55.59998 97.295134) (end 54.835 96.530154) (width 0.2) (layer "B.Cu") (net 53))
 (arc (start 67.68 106.48) (mid 67.592132 106.692132) (end 67.38 106.78) (width 0.2) (layer "B.Cu") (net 53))
 (arc (start 67.17 106.78) (mid 66.957868 106.692132) (end 66.87 106.48) (width 0.2) (layer "B.Cu") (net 53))
 (arc (start 68.28 106.08) (mid 68.192132 105.867868) (end 67.98 105.78) (width 0.2) (layer "B.Cu") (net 53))
 (arc (start 68.980006 106.78) (mid 68.485027 106.574973) (end 68.28 106.08) (width 0.2) (layer "B.Cu") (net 53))
 (arc (start 65.07 106.48) (mid 64.982132 106.692132) (end 64.77 106.78) (width 0.2) (layer "B.Cu") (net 53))
 (arc (start 66.87 106.08) (mid 66.782132 105.867868) (end 66.57 105.78) (width 0.2) (layer "B.Cu") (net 53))
 (arc (start 67.98 105.78) (mid 67.767868 105.867868) (end 67.68 106.08) (width 0.2) (layer "B.Cu") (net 53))
 (arc (start 66.57 105.78) (mid 66.357868 105.867868) (end 66.27 106.08) (width 0.2) (layer "B.Cu") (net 53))
 (arc (start 65.37 105.78) (mid 65.157868 105.867868) (end 65.07 106.08) (width 0.2) (layer "B.Cu") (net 53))
 (arc (start 65.97 106.78) (mid 65.757868 106.692132) (end 65.67 106.48) (width 0.2) (layer "B.Cu") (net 53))
 (arc (start 66.27 106.48) (mid 66.182132 106.692132) (end 65.97 106.78) (width 0.2) (layer "B.Cu") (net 53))
 (arc (start 65.67 106.08) (mid 65.582132 105.867868) (end 65.37 105.78) (width 0.2) (layer "B.Cu") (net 53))
 (segment (start 65.97 102.78) (end 70.12 102.78) (width 0.2) (layer "F.Cu") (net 50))
 (segment (start 60.14 89.96) (end 60.14 91.297918) (width 0.2) (layer "F.Cu") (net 50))
 (segment (start 60.14 92.802082) (end 60.14 93.20155) (width 0.2) (layer "F.Cu") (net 50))
 (segment (start 64.879625 102.670375) (end 64.879625 102.670374) (width 0.2) (layer "F.Cu") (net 50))
 (segment (start 64.98925 102.560749) (end 65.37 102.560749) (width 0.2) (layer "F.Cu") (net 50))
 (segment (start 65.58925 102.78) (end 65.97 102.78) (width 0.2) (layer "F.Cu") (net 50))
 (segment (start 63.33084 102.78) (end 64.77 102.78) (width 0.2) (layer "F.Cu") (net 50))
 (segment (start 61.09398 100.14578) (end 61.276 100.3278) (width 0.2) (layer "F.Cu") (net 50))
 (segment (start 59.69 89.51) (end 60.14 89.96) (width 0.2) (layer "F.Cu") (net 50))
 (segment (start 61.276 100.72516) (end 63.33084 102.78) (width 0.2) (layer "F.Cu") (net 50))
 (segment (start 60.14 91.297918) (end 60.54 91.697918) (width 0.2) (layer "F.Cu") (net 50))
 (segment (start 61.09398 94.15553) (end 61.09398 100.14578) (width 0.2) (layer "F.Cu") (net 50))
 (segment (start 61.276 100.3278) (end 61.276 100.72516) (width 0.2) (layer "F.Cu") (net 50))
 (segment (start 65.479625 102.670374) (end 65.479625 102.670375) (width 0.2) (layer "F.Cu") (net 50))
 (segment (start 60.54 91.697918) (end 60.54 92.402082) (width 0.2) (layer "F.Cu") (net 50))
 (segment (start 60.54 92.402082) (end 60.14 92.802082) (width 0.2) (layer "F.Cu") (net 50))
 (segment (start 60.14 93.20155) (end 61.09398 94.15553) (width 0.2) (layer "F.Cu") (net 50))
 (arc (start 65.479625 102.670375) (mid 65.511733 102.747892) (end 65.58925 102.78) (width 0.2) (layer "F.Cu") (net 50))
 (arc (start 64.879625 102.670374) (mid 64.911733 102.592857) (end 64.98925 102.560749) (width 0.2) (layer "F.Cu") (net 50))
 (arc (start 65.37 102.560749) (mid 65.447517 102.592857) (end 65.479625 102.670374) (width 0.2) (layer "F.Cu") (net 50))
 (arc (start 64.77 102.78) (mid 64.847517 102.747892) (end 64.879625 102.670375) (width 0.2) (layer "F.Cu") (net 50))
 (segment (start 60.644 100.3322) (end 60.82602 100.51422) (width 0.2) (layer "F.Cu") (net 51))
 (segment (start 63.144472 103.23) (end 69.29155 103.23) (width 0.2) (layer "F.Cu") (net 51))
 (segment (start 70.49445 103.684) (end 70.94845 103.23) (width 0.2) (layer "F.Cu") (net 51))
 (segment (start 69.74555 103.684) (end 70.49445 103.684) (width 0.2) (layer "F.Cu") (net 51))
 (segment (start 60.82602 100.51422) (end 60.82602 100.911548) (width 0.2) (layer "F.Cu") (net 51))
 (segment (start 60.644 94.341918) (end 60.644 100.3322) (width 0.2) (layer "F.Cu") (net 51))
 (segment (start 69.29155 103.23) (end 69.74555 103.684) (width 0.2) (layer "F.Cu") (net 51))
 (segment (start 71.67 103.23) (end 72.12 102.78) (width 0.2) (layer "F.Cu") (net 51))
 (segment (start 59.69 92.05) (end 59.69 93.387918) (width 0.2) (layer "F.Cu") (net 51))
 (segment (start 59.69 93.387918) (end 60.644 94.341918) (width 0.2) (layer "F.Cu") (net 51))
 (segment (start 60.82602 100.911548) (end 63.144472 103.23) (width 0.2) (layer "F.Cu") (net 51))
 (segment (start 70.94845 103.23) (end 71.67 103.23) (width 0.2) (layer "F.Cu") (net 51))
 (segment (start 100.33 95.25) (end 100.33 92.71) (width 0.254) (layer "B.Cu") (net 48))
 (segment (start 106.68 86.36) (end 115.57 86.36) (width 0.254) (layer "B.Cu") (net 48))
 (segment (start 100.33 92.71) (end 106.68 86.36) (width 0.254) (layer "B.Cu") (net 48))
 (segment (start 95.25 100.33) (end 100.33 95.25) (width 0.254) (layer "B.Cu") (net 48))
 (segment (start 116.84 87.63) (end 118.11 86.36) (width 0.254) (layer "B.Cu") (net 47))
 (segment (start 107.95 87.63) (end 116.84 87.63) (width 0.254) (layer "B.Cu") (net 47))
 (segment (start 101.6 96.52) (end 101.6 93.98) (width 0.254) (layer "B.Cu") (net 47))
 (segment (start 97.79 100.33) (end 101.6 96.52) (width 0.254) (layer "B.Cu") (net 47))
 (segment (start 101.6 93.98) (end 107.95 87.63) (width 0.254) (layer "B.Cu") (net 47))
 (segment (start 102.416 98.244) (end 108.766 98.244) (width 0.254) (layer "B.Cu") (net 46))
 (segment (start 100.33 100.33) (end 102.416 98.244) (width 0.254) (layer "B.Cu") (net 46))
 (segment (start 108.766 98.244) (end 120.65 86.36) (width 0.254) (layer "B.Cu") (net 46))
 (segment (start 104.502 98.698) (end 110.852 98.698) (width 0.254) (layer "B.Cu") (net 45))
 (segment (start 110.852 98.698) (end 123.19 86.36) (width 0.254) (layer "B.Cu") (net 45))
 (segment (start 102.87 100.33) (end 104.502 98.698) (width 0.254) (layer "B.Cu") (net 45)))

